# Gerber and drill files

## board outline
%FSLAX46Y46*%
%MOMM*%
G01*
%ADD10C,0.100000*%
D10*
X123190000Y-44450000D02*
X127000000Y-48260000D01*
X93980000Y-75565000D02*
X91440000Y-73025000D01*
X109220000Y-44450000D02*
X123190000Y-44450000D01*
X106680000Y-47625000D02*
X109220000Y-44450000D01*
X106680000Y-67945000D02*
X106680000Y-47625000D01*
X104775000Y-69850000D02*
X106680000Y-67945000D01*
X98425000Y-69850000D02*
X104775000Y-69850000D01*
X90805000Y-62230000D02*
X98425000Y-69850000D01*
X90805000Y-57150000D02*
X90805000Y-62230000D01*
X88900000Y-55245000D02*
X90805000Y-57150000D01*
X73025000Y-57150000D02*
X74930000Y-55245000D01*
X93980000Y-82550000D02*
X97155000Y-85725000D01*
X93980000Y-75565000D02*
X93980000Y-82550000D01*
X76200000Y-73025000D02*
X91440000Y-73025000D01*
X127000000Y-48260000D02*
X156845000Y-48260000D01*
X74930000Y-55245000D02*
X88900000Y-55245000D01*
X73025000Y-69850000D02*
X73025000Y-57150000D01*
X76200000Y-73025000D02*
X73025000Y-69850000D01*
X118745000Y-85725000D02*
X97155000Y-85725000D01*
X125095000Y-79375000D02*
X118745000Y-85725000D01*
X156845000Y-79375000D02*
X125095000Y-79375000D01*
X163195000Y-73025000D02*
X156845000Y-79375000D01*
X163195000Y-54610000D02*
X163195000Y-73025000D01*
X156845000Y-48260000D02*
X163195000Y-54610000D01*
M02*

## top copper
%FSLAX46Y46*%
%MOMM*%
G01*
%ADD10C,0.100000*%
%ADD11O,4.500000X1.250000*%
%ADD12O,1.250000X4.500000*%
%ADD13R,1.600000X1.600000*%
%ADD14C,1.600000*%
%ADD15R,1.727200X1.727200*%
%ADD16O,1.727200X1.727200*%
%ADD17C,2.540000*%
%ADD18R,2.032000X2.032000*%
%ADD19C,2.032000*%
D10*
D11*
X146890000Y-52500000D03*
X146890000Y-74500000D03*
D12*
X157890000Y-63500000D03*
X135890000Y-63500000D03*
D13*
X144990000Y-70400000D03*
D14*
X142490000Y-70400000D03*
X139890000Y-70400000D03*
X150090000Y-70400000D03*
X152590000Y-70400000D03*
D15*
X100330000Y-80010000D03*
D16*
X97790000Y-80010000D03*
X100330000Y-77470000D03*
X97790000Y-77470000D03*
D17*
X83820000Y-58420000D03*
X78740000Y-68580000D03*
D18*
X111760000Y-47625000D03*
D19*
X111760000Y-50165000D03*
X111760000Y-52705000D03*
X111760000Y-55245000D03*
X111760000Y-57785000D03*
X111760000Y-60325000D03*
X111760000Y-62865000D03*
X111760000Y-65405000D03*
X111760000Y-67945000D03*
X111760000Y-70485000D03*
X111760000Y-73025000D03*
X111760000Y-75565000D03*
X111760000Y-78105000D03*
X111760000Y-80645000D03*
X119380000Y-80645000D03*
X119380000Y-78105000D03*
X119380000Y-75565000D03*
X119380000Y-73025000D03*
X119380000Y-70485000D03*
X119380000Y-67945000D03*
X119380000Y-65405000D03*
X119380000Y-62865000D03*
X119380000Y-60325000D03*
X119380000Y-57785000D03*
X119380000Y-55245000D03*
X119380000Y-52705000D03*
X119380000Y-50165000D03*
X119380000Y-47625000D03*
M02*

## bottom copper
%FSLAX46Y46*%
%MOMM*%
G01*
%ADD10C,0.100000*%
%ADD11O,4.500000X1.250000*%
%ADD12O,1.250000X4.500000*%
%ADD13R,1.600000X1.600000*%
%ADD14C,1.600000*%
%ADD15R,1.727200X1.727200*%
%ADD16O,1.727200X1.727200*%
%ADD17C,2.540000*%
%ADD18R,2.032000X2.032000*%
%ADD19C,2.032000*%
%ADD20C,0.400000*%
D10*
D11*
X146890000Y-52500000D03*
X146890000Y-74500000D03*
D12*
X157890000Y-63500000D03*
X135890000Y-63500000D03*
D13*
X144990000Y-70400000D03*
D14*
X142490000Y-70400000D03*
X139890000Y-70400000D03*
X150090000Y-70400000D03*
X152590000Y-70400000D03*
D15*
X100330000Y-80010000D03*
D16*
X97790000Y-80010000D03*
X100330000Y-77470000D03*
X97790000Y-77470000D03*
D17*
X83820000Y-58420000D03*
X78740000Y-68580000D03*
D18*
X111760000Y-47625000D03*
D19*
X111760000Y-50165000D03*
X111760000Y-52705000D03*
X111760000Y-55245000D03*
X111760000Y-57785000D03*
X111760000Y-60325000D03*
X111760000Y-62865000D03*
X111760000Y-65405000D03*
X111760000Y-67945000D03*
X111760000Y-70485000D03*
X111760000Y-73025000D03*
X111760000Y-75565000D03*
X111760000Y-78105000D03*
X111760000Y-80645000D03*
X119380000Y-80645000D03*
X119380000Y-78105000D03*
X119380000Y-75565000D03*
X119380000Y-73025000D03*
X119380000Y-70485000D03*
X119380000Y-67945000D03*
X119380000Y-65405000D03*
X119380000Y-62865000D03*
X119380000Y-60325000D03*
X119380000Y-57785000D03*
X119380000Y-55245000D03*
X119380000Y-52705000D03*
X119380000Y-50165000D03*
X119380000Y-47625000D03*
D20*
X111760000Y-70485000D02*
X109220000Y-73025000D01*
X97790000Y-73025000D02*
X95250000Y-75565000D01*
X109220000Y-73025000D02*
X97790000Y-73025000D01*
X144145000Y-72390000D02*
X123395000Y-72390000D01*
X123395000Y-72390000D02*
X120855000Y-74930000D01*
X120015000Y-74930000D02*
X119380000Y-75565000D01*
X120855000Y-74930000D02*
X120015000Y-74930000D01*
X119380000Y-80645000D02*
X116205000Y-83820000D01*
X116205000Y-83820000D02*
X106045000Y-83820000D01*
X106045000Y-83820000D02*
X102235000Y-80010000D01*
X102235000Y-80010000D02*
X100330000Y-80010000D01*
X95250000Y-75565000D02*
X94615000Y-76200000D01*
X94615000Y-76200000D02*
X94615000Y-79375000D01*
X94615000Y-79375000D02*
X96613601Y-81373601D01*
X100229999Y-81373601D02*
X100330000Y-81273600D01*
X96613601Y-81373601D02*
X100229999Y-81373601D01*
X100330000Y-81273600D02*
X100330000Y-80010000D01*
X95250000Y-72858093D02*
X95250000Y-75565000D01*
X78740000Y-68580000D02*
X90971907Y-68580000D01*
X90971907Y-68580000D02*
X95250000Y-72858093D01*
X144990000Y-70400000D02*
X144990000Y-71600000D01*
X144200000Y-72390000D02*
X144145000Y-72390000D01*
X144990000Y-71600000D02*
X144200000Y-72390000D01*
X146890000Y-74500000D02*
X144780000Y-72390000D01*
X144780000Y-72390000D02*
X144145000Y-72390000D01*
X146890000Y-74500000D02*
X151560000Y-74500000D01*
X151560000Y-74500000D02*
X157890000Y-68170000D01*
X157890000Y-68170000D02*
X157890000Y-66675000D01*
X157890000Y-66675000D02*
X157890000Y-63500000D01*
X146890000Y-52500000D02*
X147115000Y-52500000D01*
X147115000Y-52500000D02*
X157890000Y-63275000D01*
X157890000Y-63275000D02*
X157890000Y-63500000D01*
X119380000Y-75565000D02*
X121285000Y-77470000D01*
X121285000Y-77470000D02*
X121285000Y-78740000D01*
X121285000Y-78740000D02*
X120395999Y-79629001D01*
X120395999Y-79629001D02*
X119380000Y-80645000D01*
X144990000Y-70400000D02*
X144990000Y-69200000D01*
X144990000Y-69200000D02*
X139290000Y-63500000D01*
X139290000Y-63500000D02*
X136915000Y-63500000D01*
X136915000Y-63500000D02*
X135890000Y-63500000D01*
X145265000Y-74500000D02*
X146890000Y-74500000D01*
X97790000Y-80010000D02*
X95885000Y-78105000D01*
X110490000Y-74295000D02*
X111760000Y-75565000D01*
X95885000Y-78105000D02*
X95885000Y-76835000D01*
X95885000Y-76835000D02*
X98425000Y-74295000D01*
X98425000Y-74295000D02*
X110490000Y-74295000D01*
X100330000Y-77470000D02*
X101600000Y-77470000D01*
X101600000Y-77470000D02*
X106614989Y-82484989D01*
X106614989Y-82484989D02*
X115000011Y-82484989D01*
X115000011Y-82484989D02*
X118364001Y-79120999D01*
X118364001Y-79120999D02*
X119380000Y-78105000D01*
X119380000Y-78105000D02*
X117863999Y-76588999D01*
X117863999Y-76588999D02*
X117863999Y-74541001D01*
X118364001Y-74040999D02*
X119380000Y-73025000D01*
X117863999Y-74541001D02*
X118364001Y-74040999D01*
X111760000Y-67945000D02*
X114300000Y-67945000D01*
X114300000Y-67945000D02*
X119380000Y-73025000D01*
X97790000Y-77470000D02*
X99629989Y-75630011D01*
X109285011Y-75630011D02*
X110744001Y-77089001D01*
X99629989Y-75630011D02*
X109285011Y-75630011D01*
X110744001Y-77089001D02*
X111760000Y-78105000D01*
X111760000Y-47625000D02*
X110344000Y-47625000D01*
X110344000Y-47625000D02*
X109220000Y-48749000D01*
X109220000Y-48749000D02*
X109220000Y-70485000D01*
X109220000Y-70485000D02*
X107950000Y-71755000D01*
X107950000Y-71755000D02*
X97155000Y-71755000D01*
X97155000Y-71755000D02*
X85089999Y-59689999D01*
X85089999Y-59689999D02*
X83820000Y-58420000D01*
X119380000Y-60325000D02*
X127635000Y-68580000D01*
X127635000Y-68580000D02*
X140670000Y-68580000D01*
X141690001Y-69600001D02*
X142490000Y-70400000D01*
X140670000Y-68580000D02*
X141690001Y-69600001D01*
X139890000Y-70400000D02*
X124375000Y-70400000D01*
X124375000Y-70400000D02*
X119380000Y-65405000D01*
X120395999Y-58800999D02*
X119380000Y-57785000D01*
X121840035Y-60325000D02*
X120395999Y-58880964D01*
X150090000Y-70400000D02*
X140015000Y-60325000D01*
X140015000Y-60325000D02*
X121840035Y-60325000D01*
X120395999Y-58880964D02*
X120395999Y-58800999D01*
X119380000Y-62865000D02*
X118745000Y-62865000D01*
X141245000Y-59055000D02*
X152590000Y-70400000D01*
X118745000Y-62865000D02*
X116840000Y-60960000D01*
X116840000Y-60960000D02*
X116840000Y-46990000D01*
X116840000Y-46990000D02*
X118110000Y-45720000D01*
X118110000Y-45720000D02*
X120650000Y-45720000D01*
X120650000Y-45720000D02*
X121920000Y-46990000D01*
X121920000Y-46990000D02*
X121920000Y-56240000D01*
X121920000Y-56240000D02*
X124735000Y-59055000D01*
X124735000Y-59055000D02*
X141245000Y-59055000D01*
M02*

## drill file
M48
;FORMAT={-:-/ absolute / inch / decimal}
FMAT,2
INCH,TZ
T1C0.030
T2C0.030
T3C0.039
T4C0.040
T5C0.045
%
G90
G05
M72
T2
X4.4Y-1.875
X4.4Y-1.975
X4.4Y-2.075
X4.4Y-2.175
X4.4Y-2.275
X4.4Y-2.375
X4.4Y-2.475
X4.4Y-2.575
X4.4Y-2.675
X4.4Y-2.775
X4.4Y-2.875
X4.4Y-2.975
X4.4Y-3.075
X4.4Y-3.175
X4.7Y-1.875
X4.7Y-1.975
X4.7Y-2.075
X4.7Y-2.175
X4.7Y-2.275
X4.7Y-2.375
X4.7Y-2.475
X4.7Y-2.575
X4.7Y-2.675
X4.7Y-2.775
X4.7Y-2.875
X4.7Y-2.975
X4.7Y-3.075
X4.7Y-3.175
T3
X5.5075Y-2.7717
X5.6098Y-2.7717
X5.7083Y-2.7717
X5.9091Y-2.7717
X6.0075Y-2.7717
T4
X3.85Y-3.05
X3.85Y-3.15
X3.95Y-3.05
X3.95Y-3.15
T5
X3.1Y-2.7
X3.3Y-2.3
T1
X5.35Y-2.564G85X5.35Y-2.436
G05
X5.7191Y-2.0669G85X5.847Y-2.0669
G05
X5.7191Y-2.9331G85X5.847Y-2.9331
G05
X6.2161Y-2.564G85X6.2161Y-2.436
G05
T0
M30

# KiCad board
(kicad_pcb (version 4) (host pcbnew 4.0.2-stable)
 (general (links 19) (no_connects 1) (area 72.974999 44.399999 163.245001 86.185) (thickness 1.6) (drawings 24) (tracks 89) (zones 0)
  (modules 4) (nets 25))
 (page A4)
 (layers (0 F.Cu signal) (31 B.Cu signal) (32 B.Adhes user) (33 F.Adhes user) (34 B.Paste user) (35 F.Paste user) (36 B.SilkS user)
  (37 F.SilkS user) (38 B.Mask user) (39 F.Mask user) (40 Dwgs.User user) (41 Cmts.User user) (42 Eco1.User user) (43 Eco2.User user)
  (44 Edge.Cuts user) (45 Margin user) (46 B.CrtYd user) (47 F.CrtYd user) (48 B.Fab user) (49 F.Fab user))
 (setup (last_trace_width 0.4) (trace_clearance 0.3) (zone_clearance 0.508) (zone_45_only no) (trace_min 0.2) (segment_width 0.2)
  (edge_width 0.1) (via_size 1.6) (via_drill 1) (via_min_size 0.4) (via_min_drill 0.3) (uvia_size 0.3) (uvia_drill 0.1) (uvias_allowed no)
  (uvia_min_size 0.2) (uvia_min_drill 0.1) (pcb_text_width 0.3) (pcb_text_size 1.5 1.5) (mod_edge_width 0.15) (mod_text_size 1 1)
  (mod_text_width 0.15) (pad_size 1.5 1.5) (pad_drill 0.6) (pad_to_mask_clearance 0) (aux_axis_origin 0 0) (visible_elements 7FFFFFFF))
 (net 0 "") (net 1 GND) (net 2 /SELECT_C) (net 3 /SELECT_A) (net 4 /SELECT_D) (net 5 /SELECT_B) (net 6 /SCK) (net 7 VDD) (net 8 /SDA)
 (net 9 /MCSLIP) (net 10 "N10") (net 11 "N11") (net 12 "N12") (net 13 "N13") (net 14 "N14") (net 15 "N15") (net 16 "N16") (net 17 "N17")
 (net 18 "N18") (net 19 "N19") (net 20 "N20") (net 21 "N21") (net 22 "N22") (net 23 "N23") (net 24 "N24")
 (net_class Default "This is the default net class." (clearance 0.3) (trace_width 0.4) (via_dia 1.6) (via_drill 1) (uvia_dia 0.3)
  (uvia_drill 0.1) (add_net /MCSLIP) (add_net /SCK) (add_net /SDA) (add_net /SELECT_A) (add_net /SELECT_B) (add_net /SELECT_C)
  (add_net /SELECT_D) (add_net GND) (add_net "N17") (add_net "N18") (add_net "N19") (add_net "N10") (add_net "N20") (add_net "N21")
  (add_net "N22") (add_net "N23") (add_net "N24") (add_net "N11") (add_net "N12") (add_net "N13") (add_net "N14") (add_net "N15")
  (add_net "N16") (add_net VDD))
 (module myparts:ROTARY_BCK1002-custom (layer F.Cu) (at 146.89 63.5)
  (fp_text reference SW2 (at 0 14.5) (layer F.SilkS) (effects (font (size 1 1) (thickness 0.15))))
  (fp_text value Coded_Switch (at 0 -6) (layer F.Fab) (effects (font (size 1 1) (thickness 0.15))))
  (pad 1 thru_hole oval (at 0 -11) (size 4.5 1.25) (drill oval 4 0.75) (layers *.Cu *.Mask F.SilkS) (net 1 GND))
  (pad 1 thru_hole oval (at 0 11) (size 4.5 1.25) (drill oval 4 0.75) (layers *.Cu *.Mask F.SilkS) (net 1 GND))
  (pad 1 thru_hole oval (at 11 0 90) (size 4.5 1.25) (drill oval 4 0.75) (layers *.Cu *.Mask F.SilkS) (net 1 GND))
  (pad 1 thru_hole oval (at -11 0 90) (size 4.5 1.25) (drill oval 4 0.75) (layers *.Cu *.Mask F.SilkS) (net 1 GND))
  (pad 1 thru_hole rect (at -1.9 6.9) (size 1.6 1.6) (drill 1) (layers *.Cu *.Mask F.SilkS) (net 1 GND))
  (pad 4 thru_hole circle (at -4.4 6.9) (size 1.6 1.6) (drill 1) (layers *.Cu *.Mask F.SilkS) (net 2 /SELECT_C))
  (pad 2 thru_hole circle (at -7 6.9) (size 1.6 1.6) (drill 1) (layers *.Cu *.Mask F.SilkS) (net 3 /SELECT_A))
  (pad 5 thru_hole circle (at 3.2 6.9) (size 1.6 1.6) (drill 1) (layers *.Cu *.Mask F.SilkS) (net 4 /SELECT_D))
  (pad 3 thru_hole circle (at 5.7 6.9) (size 1.6 1.6) (drill 1) (layers *.Cu *.Mask F.SilkS) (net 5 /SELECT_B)))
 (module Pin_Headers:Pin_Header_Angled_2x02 (layer F.Cu) (at 100.33 80.01 180)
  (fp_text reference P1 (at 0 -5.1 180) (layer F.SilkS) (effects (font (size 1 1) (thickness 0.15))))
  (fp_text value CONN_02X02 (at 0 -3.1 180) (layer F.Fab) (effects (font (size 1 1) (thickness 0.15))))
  (pad 1 thru_hole rect (at 0 0 180) (size 1.7272 1.7272) (drill 1.016) (layers *.Cu *.Mask F.SilkS) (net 1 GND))
  (pad 2 thru_hole oval (at 2.54 0 180) (size 1.7272 1.7272) (drill 1.016) (layers *.Cu *.Mask F.SilkS) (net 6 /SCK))
  (pad 3 thru_hole oval (at 0 2.54 180) (size 1.7272 1.7272) (drill 1.016) (layers *.Cu *.Mask F.SilkS) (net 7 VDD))
  (pad 4 thru_hole oval (at 2.54 2.54 180) (size 1.7272 1.7272) (drill 1.016) (layers *.Cu *.Mask F.SilkS) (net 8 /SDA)))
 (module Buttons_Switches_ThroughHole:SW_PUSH (layer F.Cu) (at 81.28 63.5 270)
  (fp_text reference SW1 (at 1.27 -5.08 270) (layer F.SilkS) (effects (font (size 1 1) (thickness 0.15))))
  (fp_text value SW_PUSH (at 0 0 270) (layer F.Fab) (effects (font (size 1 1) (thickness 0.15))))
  (pad 1 thru_hole circle (at -5.08 -2.54 270) (size 2.54 2.54) (drill 1.143) (layers *.Cu *.Mask F.SilkS) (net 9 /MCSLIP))
  (pad 2 thru_hole circle (at 5.08 2.54 270) (size 2.54 2.54) (drill 1.143) (layers *.Cu *.Mask F.SilkS) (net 1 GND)))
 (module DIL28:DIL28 (layer F.Cu) (at 111.76 47.625 270)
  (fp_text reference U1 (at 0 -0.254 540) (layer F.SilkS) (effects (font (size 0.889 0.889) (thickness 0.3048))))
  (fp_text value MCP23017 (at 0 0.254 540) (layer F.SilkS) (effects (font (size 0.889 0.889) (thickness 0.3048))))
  (pad 1 thru_hole rect (at 0 0 270) (size 2.032 2.032) (drill 0.762) (layers *.Cu *.Mask F.SilkS) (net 9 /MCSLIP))
  (pad 2 thru_hole circle (at 2.54 0 270) (size 2.032 2.032) (drill 0.762) (layers *.Cu *.Mask F.SilkS) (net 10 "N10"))
  (pad 3 thru_hole circle (at 5.08 0 270) (size 2.032 2.032) (drill 0.762) (layers *.Cu *.Mask F.SilkS) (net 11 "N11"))
  (pad 4 thru_hole circle (at 7.62 0 270) (size 2.032 2.032) (drill 0.762) (layers *.Cu *.Mask F.SilkS) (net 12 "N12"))
  (pad 5 thru_hole circle (at 10.16 0 270) (size 2.032 2.032) (drill 0.762) (layers *.Cu *.Mask F.SilkS) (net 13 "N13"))
  (pad 6 thru_hole circle (at 12.7 0 270) (size 2.032 2.032) (drill 0.762) (layers *.Cu *.Mask F.SilkS) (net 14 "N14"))
  (pad 7 thru_hole circle (at 15.24 0 270) (size 2.032 2.032) (drill 0.762) (layers *.Cu *.Mask F.SilkS) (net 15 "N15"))
  (pad 8 thru_hole circle (at 17.78 0 270) (size 2.032 2.032) (drill 0.762) (layers *.Cu *.Mask F.SilkS) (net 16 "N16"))
  (pad 9 thru_hole circle (at 20.32 0 270) (size 2.032 2.032) (drill 0.762) (layers *.Cu *.Mask F.SilkS) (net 7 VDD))
  (pad 10 thru_hole circle (at 22.86 0 270) (size 2.032 2.032) (drill 0.762) (layers *.Cu *.Mask F.SilkS) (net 1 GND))
  (pad 11 thru_hole circle (at 25.4 0 270) (size 2.032 2.032) (drill 0.762) (layers *.Cu *.Mask F.SilkS) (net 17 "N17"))
  (pad 12 thru_hole circle (at 27.94 0 270) (size 2.032 2.032) (drill 0.762) (layers *.Cu *.Mask F.SilkS) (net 6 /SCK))
  (pad 13 thru_hole circle (at 30.48 0 270) (size 2.032 2.032) (drill 0.762) (layers *.Cu *.Mask F.SilkS) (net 8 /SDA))
  (pad 14 thru_hole circle (at 33.02 0 270) (size 2.032 2.032) (drill 0.762) (layers *.Cu *.Mask F.SilkS) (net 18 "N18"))
  (pad 15 thru_hole circle (at 33.02 -7.62 90) (size 2.032 2.032) (drill 0.762) (layers *.Cu *.Mask F.SilkS) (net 1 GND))
  (pad 16 thru_hole circle (at 30.48 -7.62 90) (size 2.032 2.032) (drill 0.762) (layers *.Cu *.Mask F.SilkS) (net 7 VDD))
  (pad 17 thru_hole circle (at 27.94 -7.62 90) (size 2.032 2.032) (drill 0.762) (layers *.Cu *.Mask F.SilkS) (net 1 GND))
  (pad 18 thru_hole circle (at 25.4 -7.62 90) (size 2.032 2.032) (drill 0.762) (layers *.Cu *.Mask F.SilkS) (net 7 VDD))
  (pad 19 thru_hole circle (at 22.86 -7.62 90) (size 2.032 2.032) (drill 0.762) (layers *.Cu *.Mask F.SilkS) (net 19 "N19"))
  (pad 20 thru_hole circle (at 20.32 -7.62 90) (size 2.032 2.032) (drill 0.762) (layers *.Cu *.Mask F.SilkS) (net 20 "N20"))
  (pad 21 thru_hole circle (at 17.78 -7.62 90) (size 2.032 2.032) (drill 0.762) (layers *.Cu *.Mask F.SilkS) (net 3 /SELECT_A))
  (pad 22 thru_hole circle (at 15.24 -7.62 90) (size 2.032 2.032) (drill 0.762) (layers *.Cu *.Mask F.SilkS) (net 5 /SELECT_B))
  (pad 23 thru_hole circle (at 12.7 -7.62 90) (size 2.032 2.032) (drill 0.762) (layers *.Cu *.Mask F.SilkS) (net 2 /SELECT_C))
  (pad 24 thru_hole circle (at 10.16 -7.62 90) (size 2.032 2.032) (drill 0.762) (layers *.Cu *.Mask F.SilkS) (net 4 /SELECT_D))
  (pad 25 thru_hole circle (at 7.62 -7.62 90) (size 2.032 2.032) (drill 0.762) (layers *.Cu *.Mask F.SilkS) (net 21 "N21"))
  (pad 26 thru_hole circle (at 5.08 -7.62 90) (size 2.032 2.032) (drill 0.762) (layers *.Cu *.Mask F.SilkS) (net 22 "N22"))
  (pad 27 thru_hole circle (at 2.54 -7.62 90) (size 2.032 2.032) (drill 0.762) (layers *.Cu *.Mask F.SilkS) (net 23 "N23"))
  (pad 28 thru_hole circle (at 0 -7.62 90) (size 2.032 2.032) (drill 0.762) (layers *.Cu *.Mask F.SilkS) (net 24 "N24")))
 (gr_line (start 123.19 44.45) (end 127 48.26) (layer Edge.Cuts) (width 0.1))
 (gr_line (start 93.98 75.565) (end 91.44 73.025) (layer Edge.Cuts) (width 0.1))
 (gr_line (start 109.22 44.45) (end 123.19 44.45) (layer Edge.Cuts) (width 0.1))
 (gr_line (start 106.68 47.625) (end 109.22 44.45) (layer Edge.Cuts) (width 0.1))
 (gr_line (start 106.68 67.945) (end 106.68 47.625) (layer Edge.Cuts) (width 0.1))
 (gr_line (start 104.775 69.85) (end 106.68 67.945) (layer Edge.Cuts) (width 0.1))
 (gr_line (start 98.425 69.85) (end 104.775 69.85) (layer Edge.Cuts) (width 0.1))
 (gr_line (start 90.805 62.23) (end 98.425 69.85) (layer Edge.Cuts) (width 0.1))
 (gr_line (start 90.805 57.15) (end 90.805 62.23) (layer Edge.Cuts) (width 0.1))
 (gr_line (start 88.9 55.245) (end 90.805 57.15) (layer Edge.Cuts) (width 0.1))
 (gr_line (start 73.025 57.15) (end 74.93 55.245) (layer Edge.Cuts) (width 0.1))
 (gr_line (start 93.98 82.55) (end 97.155 85.725) (layer Edge.Cuts) (width 0.1))
 (gr_line (start 93.98 75.565) (end 93.98 82.55) (layer Edge.Cuts) (width 0.1))
 (gr_line (start 76.2 73.025) (end 91.44 73.025) (layer Edge.Cuts) (width 0.1))
 (gr_line (start 127 48.26) (end 156.845 48.26) (layer Edge.Cuts) (width 0.1))
 (gr_line (start 74.93 55.245) (end 88.9 55.245) (layer Edge.Cuts) (width 0.1))
 (gr_line (start 73.025 69.85) (end 73.025 57.15) (layer Edge.Cuts) (width 0.1))
 (gr_line (start 76.2 73.025) (end 73.025 69.85) (layer Edge.Cuts) (width 0.1))
 (gr_line (start 118.745 85.725) (end 97.155 85.725) (layer Edge.Cuts) (width 0.1))
 (gr_line (start 125.095 79.375) (end 118.745 85.725) (layer Edge.Cuts) (width 0.1))
 (gr_line (start 156.845 79.375) (end 125.095 79.375) (layer Edge.Cuts) (width 0.1))
 (gr_line (start 163.195 73.025) (end 156.845 79.375) (layer Edge.Cuts) (width 0.1))
 (gr_line (start 163.195 54.61) (end 163.195 73.025) (layer Edge.Cuts) (width 0.1))
 (gr_line (start 156.845 48.26) (end 163.195 54.61) (layer Edge.Cuts) (width 0.1))
 (segment (start 111.76 70.485) (end 109.22 73.025) (width 0.4) (layer B.Cu) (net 1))
 (segment (start 97.79 73.025) (end 95.25 75.565) (width 0.4) (layer B.Cu) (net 1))
 (segment (start 109.22 73.025) (end 97.79 73.025) (width 0.4) (layer B.Cu) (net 1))
 (segment (start 144.145 72.39) (end 123.395 72.39) (width 0.4) (layer B.Cu) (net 1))
 (segment (start 123.395 72.39) (end 120.855 74.93) (width 0.4) (layer B.Cu) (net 1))
 (segment (start 120.015 74.93) (end 119.38 75.565) (width 0.4) (layer B.Cu) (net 1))
 (segment (start 120.855 74.93) (end 120.015 74.93) (width 0.4) (layer B.Cu) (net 1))
 (segment (start 119.38 80.645) (end 116.205 83.82) (width 0.4) (layer B.Cu) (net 1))
 (segment (start 116.205 83.82) (end 106.045 83.82) (width 0.4) (layer B.Cu) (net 1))
 (segment (start 106.045 83.82) (end 102.235 80.01) (width 0.4) (layer B.Cu) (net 1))
 (segment (start 102.235 80.01) (end 100.33 80.01) (width 0.4) (layer B.Cu) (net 1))
 (segment (start 95.25 75.565) (end 94.615 76.2) (width 0.4) (layer B.Cu) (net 1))
 (segment (start 94.615 76.2) (end 94.615 79.375) (width 0.4) (layer B.Cu) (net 1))
 (segment (start 94.615 79.375) (end 96.613601 81.373601) (width 0.4) (layer B.Cu) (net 1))
 (segment (start 100.229999 81.373601) (end 100.33 81.2736) (width 0.4) (layer B.Cu) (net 1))
 (segment (start 96.613601 81.373601) (end 100.229999 81.373601) (width 0.4) (layer B.Cu) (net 1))
 (segment (start 100.33 81.2736) (end 100.33 80.01) (width 0.4) (layer B.Cu) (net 1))
 (segment (start 95.25 72.858093) (end 95.25 75.565) (width 0.4) (layer B.Cu) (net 1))
 (segment (start 78.74 68.58) (end 90.971907 68.58) (width 0.4) (layer B.Cu) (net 1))
 (segment (start 90.971907 68.58) (end 95.25 72.858093) (width 0.4) (layer B.Cu) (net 1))
 (segment (start 144.99 70.4) (end 144.99 71.6) (width 0.4) (layer B.Cu) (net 1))
 (segment (start 144.2 72.39) (end 144.145 72.39) (width 0.4) (layer B.Cu) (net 1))
 (segment (start 144.99 71.6) (end 144.2 72.39) (width 0.4) (layer B.Cu) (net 1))
 (segment (start 146.89 74.5) (end 144.78 72.39) (width 0.4) (layer B.Cu) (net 1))
 (segment (start 144.78 72.39) (end 144.145 72.39) (width 0.4) (layer B.Cu) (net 1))
 (segment (start 146.89 74.5) (end 151.56 74.5) (width 0.4) (layer B.Cu) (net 1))
 (segment (start 151.56 74.5) (end 157.89 68.17) (width 0.4) (layer B.Cu) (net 1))
 (segment (start 157.89 68.17) (end 157.89 66.675) (width 0.4) (layer B.Cu) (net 1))
 (segment (start 157.89 66.675) (end 157.89 63.5) (width 0.4) (layer B.Cu) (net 1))
 (segment (start 146.89 52.5) (end 147.115 52.5) (width 0.4) (layer B.Cu) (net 1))
 (segment (start 147.115 52.5) (end 157.89 63.275) (width 0.4) (layer B.Cu) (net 1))
 (segment (start 157.89 63.275) (end 157.89 63.5) (width 0.4) (layer B.Cu) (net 1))
 (segment (start 119.38 75.565) (end 121.285 77.47) (width 0.4) (layer B.Cu) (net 1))
 (segment (start 121.285 77.47) (end 121.285 78.74) (width 0.4) (layer B.Cu) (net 1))
 (segment (start 121.285 78.74) (end 120.395999 79.629001) (width 0.4) (layer B.Cu) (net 1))
 (segment (start 120.395999 79.629001) (end 119.38 80.645) (width 0.4) (layer B.Cu) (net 1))
 (segment (start 144.99 70.4) (end 144.99 69.2) (width 0.4) (layer B.Cu) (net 1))
 (segment (start 144.99 69.2) (end 139.29 63.5) (width 0.4) (layer B.Cu) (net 1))
 (segment (start 139.29 63.5) (end 136.915 63.5) (width 0.4) (layer B.Cu) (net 1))
 (segment (start 136.915 63.5) (end 135.89 63.5) (width 0.4) (layer B.Cu) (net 1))
 (segment (start 145.265 74.5) (end 146.89 74.5) (width 0.4) (layer B.Cu) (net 1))
 (segment (start 97.79 80.01) (end 95.885 78.105) (width 0.4) (layer B.Cu) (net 6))
 (segment (start 110.49 74.295) (end 111.76 75.565) (width 0.4) (layer B.Cu) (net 6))
 (segment (start 95.885 78.105) (end 95.885 76.835) (width 0.4) (layer B.Cu) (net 6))
 (segment (start 95.885 76.835) (end 98.425 74.295) (width 0.4) (layer B.Cu) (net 6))
 (segment (start 98.425 74.295) (end 110.49 74.295) (width 0.4) (layer B.Cu) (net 6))
 (segment (start 100.33 77.47) (end 101.6 77.47) (width 0.4) (layer B.Cu) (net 7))
 (segment (start 101.6 77.47) (end 106.614989 82.484989) (width 0.4) (layer B.Cu) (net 7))
 (segment (start 106.614989 82.484989) (end 115.000011 82.484989) (width 0.4) (layer B.Cu) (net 7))
 (segment (start 115.000011 82.484989) (end 118.364001 79.120999) (width 0.4) (layer B.Cu) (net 7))
 (segment (start 118.364001 79.120999) (end 119.38 78.105) (width 0.4) (layer B.Cu) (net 7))
 (segment (start 119.38 78.105) (end 117.863999 76.588999) (width 0.4) (layer B.Cu) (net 7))
 (segment (start 117.863999 76.588999) (end 117.863999 74.541001) (width 0.4) (layer B.Cu) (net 7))
 (segment (start 118.364001 74.040999) (end 119.38 73.025) (width 0.4) (layer B.Cu) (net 7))
 (segment (start 117.863999 74.541001) (end 118.364001 74.040999) (width 0.4) (layer B.Cu) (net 7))
 (segment (start 111.76 67.945) (end 114.3 67.945) (width 0.4) (layer B.Cu) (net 7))
 (segment (start 114.3 67.945) (end 119.38 73.025) (width 0.4) (layer B.Cu) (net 7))
 (segment (start 97.79 77.47) (end 99.629989 75.630011) (width 0.4) (layer B.Cu) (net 8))
 (segment (start 109.285011 75.630011) (end 110.744001 77.089001) (width 0.4) (layer B.Cu) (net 8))
 (segment (start 99.629989 75.630011) (end 109.285011 75.630011) (width 0.4) (layer B.Cu) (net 8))
 (segment (start 110.744001 77.089001) (end 111.76 78.105) (width 0.4) (layer B.Cu) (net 8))
 (segment (start 111.76 47.625) (end 110.344 47.625) (width 0.4) (layer B.Cu) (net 9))
 (segment (start 110.344 47.625) (end 109.22 48.749) (width 0.4) (layer B.Cu) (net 9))
 (segment (start 109.22 48.749) (end 109.22 70.485) (width 0.4) (layer B.Cu) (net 9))
 (segment (start 109.22 70.485) (end 107.95 71.755) (width 0.4) (layer B.Cu) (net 9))
 (segment (start 107.95 71.755) (end 97.155 71.755) (width 0.4) (layer B.Cu) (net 9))
 (segment (start 97.155 71.755) (end 85.089999 59.689999) (width 0.4) (layer B.Cu) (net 9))
 (segment (start 85.089999 59.689999) (end 83.82 58.42) (width 0.4) (layer B.Cu) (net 9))
 (segment (start 119.38 60.325) (end 127.635 68.58) (width 0.4) (layer B.Cu) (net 2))
 (segment (start 127.635 68.58) (end 140.67 68.58) (width 0.4) (layer B.Cu) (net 2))
 (segment (start 141.690001 69.600001) (end 142.49 70.4) (width 0.4) (layer B.Cu) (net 2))
 (segment (start 140.67 68.58) (end 141.690001 69.600001) (width 0.4) (layer B.Cu) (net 2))
 (segment (start 139.89 70.4) (end 124.375 70.4) (width 0.4) (layer B.Cu) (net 3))
 (segment (start 124.375 70.4) (end 119.38 65.405) (width 0.4) (layer B.Cu) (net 3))
 (segment (start 120.395999 58.800999) (end 119.38 57.785) (width 0.4) (layer B.Cu) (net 4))
 (segment (start 121.840035 60.325) (end 120.395999 58.880964) (width 0.4) (layer B.Cu) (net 4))
 (segment (start 150.09 70.4) (end 140.015 60.325) (width 0.4) (layer B.Cu) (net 4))
 (segment (start 140.015 60.325) (end 121.840035 60.325) (width 0.4) (layer B.Cu) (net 4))
 (segment (start 120.395999 58.880964) (end 120.395999 58.800999) (width 0.4) (layer B.Cu) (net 4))
 (segment (start 119.38 62.865) (end 118.745 62.865) (width 0.4) (layer B.Cu) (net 5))
 (segment (start 141.245 59.055) (end 152.59 70.4) (width 0.4) (layer B.Cu) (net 5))
 (segment (start 118.745 62.865) (end 116.84 60.96) (width 0.4) (layer B.Cu) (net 5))
 (segment (start 116.84 60.96) (end 116.84 46.99) (width 0.4) (layer B.Cu) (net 5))
 (segment (start 116.84 46.99) (end 118.11 45.72) (width 0.4) (layer B.Cu) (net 5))
 (segment (start 118.11 45.72) (end 120.65 45.72) (width 0.4) (layer B.Cu) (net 5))
 (segment (start 120.65 45.72) (end 121.92 46.99) (width 0.4) (layer B.Cu) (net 5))
 (segment (start 121.92 46.99) (end 121.92 56.24) (width 0.4) (layer B.Cu) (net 5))
 (segment (start 121.92 56.24) (end 124.735 59.055) (width 0.4) (layer B.Cu) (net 5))
 (segment (start 124.735 59.055) (end 141.245 59.055) (width 0.4) (layer B.Cu) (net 5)))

